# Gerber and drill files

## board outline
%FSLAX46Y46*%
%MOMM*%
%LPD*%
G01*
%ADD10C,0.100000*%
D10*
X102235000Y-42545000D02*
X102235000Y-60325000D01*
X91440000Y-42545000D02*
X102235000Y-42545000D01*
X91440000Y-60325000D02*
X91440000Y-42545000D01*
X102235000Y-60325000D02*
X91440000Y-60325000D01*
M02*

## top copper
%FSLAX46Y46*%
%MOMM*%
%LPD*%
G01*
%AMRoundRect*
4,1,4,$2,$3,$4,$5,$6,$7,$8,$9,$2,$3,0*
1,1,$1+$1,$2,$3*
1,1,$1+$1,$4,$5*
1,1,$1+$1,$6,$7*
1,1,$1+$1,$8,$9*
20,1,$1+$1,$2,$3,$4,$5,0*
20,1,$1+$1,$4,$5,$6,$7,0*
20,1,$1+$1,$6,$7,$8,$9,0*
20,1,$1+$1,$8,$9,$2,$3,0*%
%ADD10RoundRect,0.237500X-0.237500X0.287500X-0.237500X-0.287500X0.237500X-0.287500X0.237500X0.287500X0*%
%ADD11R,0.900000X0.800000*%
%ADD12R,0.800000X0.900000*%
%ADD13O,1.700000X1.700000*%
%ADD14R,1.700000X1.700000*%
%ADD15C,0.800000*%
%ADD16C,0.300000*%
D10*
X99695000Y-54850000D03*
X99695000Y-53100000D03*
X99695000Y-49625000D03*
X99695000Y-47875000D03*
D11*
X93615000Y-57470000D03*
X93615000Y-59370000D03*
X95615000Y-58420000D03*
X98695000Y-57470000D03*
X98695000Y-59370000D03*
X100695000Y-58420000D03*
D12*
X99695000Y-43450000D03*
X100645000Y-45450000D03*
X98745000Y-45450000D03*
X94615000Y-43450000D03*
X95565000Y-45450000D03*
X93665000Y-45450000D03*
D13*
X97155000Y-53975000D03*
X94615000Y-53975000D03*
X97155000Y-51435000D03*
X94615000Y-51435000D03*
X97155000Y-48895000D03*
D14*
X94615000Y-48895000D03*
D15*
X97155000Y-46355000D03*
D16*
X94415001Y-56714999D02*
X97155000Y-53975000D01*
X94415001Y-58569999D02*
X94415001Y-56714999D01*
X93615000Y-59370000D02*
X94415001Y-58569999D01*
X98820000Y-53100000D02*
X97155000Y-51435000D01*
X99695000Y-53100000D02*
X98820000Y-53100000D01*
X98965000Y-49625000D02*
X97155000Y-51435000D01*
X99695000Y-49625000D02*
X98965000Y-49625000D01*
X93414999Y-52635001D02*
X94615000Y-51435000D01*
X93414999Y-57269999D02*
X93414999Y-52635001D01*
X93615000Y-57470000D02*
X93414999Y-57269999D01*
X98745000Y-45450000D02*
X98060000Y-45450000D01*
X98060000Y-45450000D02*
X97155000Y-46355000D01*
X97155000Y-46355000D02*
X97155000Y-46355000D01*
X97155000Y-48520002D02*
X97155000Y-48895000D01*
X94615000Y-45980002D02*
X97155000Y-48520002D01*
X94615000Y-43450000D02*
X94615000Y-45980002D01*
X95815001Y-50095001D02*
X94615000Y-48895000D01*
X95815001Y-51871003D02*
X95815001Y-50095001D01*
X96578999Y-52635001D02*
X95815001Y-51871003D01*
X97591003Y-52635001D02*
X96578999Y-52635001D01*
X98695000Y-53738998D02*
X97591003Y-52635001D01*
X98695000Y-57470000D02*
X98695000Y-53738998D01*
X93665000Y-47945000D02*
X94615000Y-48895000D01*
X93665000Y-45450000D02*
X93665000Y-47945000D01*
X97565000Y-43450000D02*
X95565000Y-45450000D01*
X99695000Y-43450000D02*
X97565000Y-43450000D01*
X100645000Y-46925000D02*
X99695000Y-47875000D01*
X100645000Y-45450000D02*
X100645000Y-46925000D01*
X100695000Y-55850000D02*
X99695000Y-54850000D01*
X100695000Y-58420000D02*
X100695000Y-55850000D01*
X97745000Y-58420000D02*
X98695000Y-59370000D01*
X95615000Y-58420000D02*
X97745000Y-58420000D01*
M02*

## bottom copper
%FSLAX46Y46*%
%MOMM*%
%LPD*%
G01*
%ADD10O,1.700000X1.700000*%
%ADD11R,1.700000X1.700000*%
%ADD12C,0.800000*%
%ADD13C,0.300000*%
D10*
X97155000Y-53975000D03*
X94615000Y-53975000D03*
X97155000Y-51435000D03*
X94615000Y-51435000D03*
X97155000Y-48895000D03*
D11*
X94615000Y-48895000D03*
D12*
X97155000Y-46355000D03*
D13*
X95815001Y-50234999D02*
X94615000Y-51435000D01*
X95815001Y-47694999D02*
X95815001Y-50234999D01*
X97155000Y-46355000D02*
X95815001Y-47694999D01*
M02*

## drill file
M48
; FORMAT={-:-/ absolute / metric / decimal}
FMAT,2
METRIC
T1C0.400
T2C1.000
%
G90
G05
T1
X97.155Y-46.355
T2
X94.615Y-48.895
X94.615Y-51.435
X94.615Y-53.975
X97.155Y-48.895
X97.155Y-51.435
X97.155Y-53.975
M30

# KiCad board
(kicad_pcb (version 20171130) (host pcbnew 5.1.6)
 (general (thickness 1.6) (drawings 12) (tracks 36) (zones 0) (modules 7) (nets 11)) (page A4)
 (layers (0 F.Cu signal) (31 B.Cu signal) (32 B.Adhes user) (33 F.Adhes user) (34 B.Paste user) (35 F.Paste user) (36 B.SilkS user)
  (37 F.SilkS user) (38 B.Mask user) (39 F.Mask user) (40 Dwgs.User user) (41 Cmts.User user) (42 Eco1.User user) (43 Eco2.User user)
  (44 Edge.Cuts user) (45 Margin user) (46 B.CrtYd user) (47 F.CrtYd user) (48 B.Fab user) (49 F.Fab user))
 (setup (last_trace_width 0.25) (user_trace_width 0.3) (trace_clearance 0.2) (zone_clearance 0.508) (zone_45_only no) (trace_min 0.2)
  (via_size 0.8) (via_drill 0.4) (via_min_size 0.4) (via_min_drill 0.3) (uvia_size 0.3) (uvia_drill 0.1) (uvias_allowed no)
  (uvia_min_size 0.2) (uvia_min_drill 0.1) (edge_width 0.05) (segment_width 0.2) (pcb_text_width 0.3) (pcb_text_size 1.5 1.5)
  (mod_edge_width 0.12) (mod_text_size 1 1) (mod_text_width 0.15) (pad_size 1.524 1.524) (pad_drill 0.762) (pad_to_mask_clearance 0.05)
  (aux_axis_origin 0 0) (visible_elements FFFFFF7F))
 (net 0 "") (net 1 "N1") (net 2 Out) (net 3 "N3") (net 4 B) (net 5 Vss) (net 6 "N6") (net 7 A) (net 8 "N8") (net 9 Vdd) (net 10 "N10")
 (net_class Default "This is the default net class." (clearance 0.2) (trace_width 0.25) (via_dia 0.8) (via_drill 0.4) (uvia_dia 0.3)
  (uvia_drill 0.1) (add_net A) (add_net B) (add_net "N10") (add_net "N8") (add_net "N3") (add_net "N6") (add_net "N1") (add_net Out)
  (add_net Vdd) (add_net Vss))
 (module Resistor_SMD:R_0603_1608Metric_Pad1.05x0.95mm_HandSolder (layer F.Cu) (at 99.695 53.975 270)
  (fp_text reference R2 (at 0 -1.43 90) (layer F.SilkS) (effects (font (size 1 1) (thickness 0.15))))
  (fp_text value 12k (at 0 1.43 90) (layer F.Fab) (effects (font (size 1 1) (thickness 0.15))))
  (pad 2 smd roundrect (at 0.875 0 270) (size 1.05 0.95) (layers F.Cu F.Paste F.Mask) (roundrect_rratio 0.25) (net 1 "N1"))
  (pad 1 smd roundrect (at -0.875 0 270) (size 1.05 0.95) (layers F.Cu F.Paste F.Mask) (roundrect_rratio 0.25) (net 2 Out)))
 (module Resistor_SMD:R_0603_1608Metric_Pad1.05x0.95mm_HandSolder (layer F.Cu) (at 99.695 48.75 270)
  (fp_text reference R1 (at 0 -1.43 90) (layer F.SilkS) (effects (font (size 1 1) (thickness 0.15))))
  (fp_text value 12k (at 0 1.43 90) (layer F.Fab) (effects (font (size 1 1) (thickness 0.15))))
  (pad 2 smd roundrect (at 0.875 0 270) (size 1.05 0.95) (layers F.Cu F.Paste F.Mask) (roundrect_rratio 0.25) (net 2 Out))
  (pad 1 smd roundrect (at -0.875 0 270) (size 1.05 0.95) (layers F.Cu F.Paste F.Mask) (roundrect_rratio 0.25) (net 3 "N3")))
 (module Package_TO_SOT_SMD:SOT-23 (layer F.Cu) (at 94.615 58.42)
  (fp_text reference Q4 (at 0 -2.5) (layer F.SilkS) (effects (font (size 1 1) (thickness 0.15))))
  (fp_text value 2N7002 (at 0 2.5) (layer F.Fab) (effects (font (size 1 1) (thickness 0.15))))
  (pad 1 smd rect (at -1 -0.95) (size 0.9 0.8) (layers F.Cu F.Paste F.Mask) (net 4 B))
  (pad 2 smd rect (at -1 0.95) (size 0.9 0.8) (layers F.Cu F.Paste F.Mask) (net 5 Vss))
  (pad 3 smd rect (at 1 0) (size 0.9 0.8) (layers F.Cu F.Paste F.Mask) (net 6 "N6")))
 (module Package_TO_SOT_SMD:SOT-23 (layer F.Cu) (at 99.695 58.42)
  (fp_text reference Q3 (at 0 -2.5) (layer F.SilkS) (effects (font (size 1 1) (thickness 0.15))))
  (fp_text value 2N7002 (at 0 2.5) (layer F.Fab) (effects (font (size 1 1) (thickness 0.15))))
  (pad 1 smd rect (at -1 -0.95) (size 0.9 0.8) (layers F.Cu F.Paste F.Mask) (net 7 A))
  (pad 2 smd rect (at -1 0.95) (size 0.9 0.8) (layers F.Cu F.Paste F.Mask) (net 6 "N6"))
  (pad 3 smd rect (at 1 0) (size 0.9 0.8) (layers F.Cu F.Paste F.Mask) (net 1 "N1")))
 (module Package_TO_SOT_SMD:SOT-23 (layer F.Cu) (at 99.695 44.45 90)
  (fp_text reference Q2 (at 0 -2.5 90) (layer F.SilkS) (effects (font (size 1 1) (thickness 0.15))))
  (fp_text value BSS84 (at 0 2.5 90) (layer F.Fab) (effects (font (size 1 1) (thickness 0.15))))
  (pad 3 smd rect (at 1 0 90) (size 0.9 0.8) (layers F.Cu F.Paste F.Mask) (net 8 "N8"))
  (pad 2 smd rect (at -1 0.95 90) (size 0.9 0.8) (layers F.Cu F.Paste F.Mask) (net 3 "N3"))
  (pad 1 smd rect (at -1 -0.95 90) (size 0.9 0.8) (layers F.Cu F.Paste F.Mask) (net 4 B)))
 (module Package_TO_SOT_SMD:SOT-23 (layer F.Cu) (at 94.615 44.45 90)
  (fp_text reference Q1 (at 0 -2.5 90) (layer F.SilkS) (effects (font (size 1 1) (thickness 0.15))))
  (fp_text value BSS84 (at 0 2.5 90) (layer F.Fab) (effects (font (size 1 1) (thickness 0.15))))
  (pad 3 smd rect (at 1 0 90) (size 0.9 0.8) (layers F.Cu F.Paste F.Mask) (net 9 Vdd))
  (pad 2 smd rect (at -1 0.95 90) (size 0.9 0.8) (layers F.Cu F.Paste F.Mask) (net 8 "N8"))
  (pad 1 smd rect (at -1 -0.95 90) (size 0.9 0.8) (layers F.Cu F.Paste F.Mask) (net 7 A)))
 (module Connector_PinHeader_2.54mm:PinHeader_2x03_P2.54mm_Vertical (layer F.Cu) (at 94.615 48.895)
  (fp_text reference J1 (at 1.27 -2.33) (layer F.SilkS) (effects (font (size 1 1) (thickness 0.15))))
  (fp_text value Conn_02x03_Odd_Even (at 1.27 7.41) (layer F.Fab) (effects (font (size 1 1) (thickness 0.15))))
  (pad 6 thru_hole oval (at 2.54 5.08) (size 1.7 1.7) (drill 1) (layers *.Cu *.Mask) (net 5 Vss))
  (pad 5 thru_hole oval (at 0 5.08) (size 1.7 1.7) (drill 1) (layers *.Cu *.Mask) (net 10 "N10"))
  (pad 4 thru_hole oval (at 2.54 2.54) (size 1.7 1.7) (drill 1) (layers *.Cu *.Mask) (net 2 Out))
  (pad 3 thru_hole oval (at 0 2.54) (size 1.7 1.7) (drill 1) (layers *.Cu *.Mask) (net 4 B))
  (pad 2 thru_hole oval (at 2.54 0) (size 1.7 1.7) (drill 1) (layers *.Cu *.Mask) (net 9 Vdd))
  (pad 1 thru_hole rect (at 0 0) (size 1.7 1.7) (drill 1) (layers *.Cu *.Mask) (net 7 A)))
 (gr_line (start 102.235 42.545) (end 102.235 60.325) (layer Edge.Cuts) (width 0.1))
 (gr_line (start 91.44 42.545) (end 102.235 42.545) (layer Edge.Cuts) (width 0.1))
 (gr_line (start 91.44 60.325) (end 91.44 42.545) (layer Edge.Cuts) (width 0.1))
 (gr_line (start 102.235 60.325) (end 91.44 60.325) (layer Edge.Cuts) (width 0.1))
 (segment (start 94.415001 56.714999) (end 97.155 53.975) (width 0.3) (layer F.Cu) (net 5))
 (segment (start 94.415001 58.569999) (end 94.415001 56.714999) (width 0.3) (layer F.Cu) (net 5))
 (segment (start 93.615 59.37) (end 94.415001 58.569999) (width 0.3) (layer F.Cu) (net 5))
 (segment (start 98.82 53.1) (end 97.155 51.435) (width 0.3) (layer F.Cu) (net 2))
 (segment (start 99.695 53.1) (end 98.82 53.1) (width 0.3) (layer F.Cu) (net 2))
 (segment (start 98.965 49.625) (end 97.155 51.435) (width 0.3) (layer F.Cu) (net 2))
 (segment (start 99.695 49.625) (end 98.965 49.625) (width 0.3) (layer F.Cu) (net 2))
 (segment (start 93.414999 52.635001) (end 94.615 51.435) (width 0.3) (layer F.Cu) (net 4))
 (segment (start 93.414999 57.269999) (end 93.414999 52.635001) (width 0.3) (layer F.Cu) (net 4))
 (segment (start 93.615 57.47) (end 93.414999 57.269999) (width 0.3) (layer F.Cu) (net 4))
 (segment (start 98.745 45.45) (end 98.06 45.45) (width 0.3) (layer F.Cu) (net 4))
 (segment (start 98.06 45.45) (end 97.155 46.355) (width 0.3) (layer F.Cu) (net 4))
 (segment (start 97.155 46.355) (end 97.155 46.355) (width 0.3) (layer F.Cu) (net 4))
 (via (at 97.155 46.355) (size 0.8) (drill 0.4) (layers F.Cu B.Cu) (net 4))
 (segment (start 95.815001 50.234999) (end 94.615 51.435) (width 0.3) (layer B.Cu) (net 4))
 (segment (start 95.815001 47.694999) (end 95.815001 50.234999) (width 0.3) (layer B.Cu) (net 4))
 (segment (start 97.155 46.355) (end 95.815001 47.694999) (width 0.3) (layer B.Cu) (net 4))
 (segment (start 97.155 48.520002) (end 97.155 48.895) (width 0.3) (layer F.Cu) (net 9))
 (segment (start 94.615 45.980002) (end 97.155 48.520002) (width 0.3) (layer F.Cu) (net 9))
 (segment (start 94.615 43.45) (end 94.615 45.980002) (width 0.3) (layer F.Cu) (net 9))
 (segment (start 95.815001 50.095001) (end 94.615 48.895) (width 0.3) (layer F.Cu) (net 7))
 (segment (start 95.815001 51.871003) (end 95.815001 50.095001) (width 0.3) (layer F.Cu) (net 7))
 (segment (start 96.578999 52.635001) (end 95.815001 51.871003) (width 0.3) (layer F.Cu) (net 7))
 (segment (start 97.591003 52.635001) (end 96.578999 52.635001) (width 0.3) (layer F.Cu) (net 7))
 (segment (start 98.695 53.738998) (end 97.591003 52.635001) (width 0.3) (layer F.Cu) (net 7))
 (segment (start 98.695 57.47) (end 98.695 53.738998) (width 0.3) (layer F.Cu) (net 7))
 (segment (start 93.665 47.945) (end 94.615 48.895) (width 0.3) (layer F.Cu) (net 7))
 (segment (start 93.665 45.45) (end 93.665 47.945) (width 0.3) (layer F.Cu) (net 7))
 (segment (start 97.565 43.45) (end 95.565 45.45) (width 0.3) (layer F.Cu) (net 8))
 (segment (start 99.695 43.45) (end 97.565 43.45) (width 0.3) (layer F.Cu) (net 8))
 (segment (start 100.645 46.925) (end 99.695 47.875) (width 0.3) (layer F.Cu) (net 3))
 (segment (start 100.645 45.45) (end 100.645 46.925) (width 0.3) (layer F.Cu) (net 3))
 (segment (start 100.695 55.85) (end 99.695 54.85) (width 0.3) (layer F.Cu) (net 1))
 (segment (start 100.695 58.42) (end 100.695 55.85) (width 0.3) (layer F.Cu) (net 1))
 (segment (start 97.745 58.42) (end 98.695 59.37) (width 0.3) (layer F.Cu) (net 6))
 (segment (start 95.615 58.42) (end 97.745 58.42) (width 0.3) (layer F.Cu) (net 6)))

